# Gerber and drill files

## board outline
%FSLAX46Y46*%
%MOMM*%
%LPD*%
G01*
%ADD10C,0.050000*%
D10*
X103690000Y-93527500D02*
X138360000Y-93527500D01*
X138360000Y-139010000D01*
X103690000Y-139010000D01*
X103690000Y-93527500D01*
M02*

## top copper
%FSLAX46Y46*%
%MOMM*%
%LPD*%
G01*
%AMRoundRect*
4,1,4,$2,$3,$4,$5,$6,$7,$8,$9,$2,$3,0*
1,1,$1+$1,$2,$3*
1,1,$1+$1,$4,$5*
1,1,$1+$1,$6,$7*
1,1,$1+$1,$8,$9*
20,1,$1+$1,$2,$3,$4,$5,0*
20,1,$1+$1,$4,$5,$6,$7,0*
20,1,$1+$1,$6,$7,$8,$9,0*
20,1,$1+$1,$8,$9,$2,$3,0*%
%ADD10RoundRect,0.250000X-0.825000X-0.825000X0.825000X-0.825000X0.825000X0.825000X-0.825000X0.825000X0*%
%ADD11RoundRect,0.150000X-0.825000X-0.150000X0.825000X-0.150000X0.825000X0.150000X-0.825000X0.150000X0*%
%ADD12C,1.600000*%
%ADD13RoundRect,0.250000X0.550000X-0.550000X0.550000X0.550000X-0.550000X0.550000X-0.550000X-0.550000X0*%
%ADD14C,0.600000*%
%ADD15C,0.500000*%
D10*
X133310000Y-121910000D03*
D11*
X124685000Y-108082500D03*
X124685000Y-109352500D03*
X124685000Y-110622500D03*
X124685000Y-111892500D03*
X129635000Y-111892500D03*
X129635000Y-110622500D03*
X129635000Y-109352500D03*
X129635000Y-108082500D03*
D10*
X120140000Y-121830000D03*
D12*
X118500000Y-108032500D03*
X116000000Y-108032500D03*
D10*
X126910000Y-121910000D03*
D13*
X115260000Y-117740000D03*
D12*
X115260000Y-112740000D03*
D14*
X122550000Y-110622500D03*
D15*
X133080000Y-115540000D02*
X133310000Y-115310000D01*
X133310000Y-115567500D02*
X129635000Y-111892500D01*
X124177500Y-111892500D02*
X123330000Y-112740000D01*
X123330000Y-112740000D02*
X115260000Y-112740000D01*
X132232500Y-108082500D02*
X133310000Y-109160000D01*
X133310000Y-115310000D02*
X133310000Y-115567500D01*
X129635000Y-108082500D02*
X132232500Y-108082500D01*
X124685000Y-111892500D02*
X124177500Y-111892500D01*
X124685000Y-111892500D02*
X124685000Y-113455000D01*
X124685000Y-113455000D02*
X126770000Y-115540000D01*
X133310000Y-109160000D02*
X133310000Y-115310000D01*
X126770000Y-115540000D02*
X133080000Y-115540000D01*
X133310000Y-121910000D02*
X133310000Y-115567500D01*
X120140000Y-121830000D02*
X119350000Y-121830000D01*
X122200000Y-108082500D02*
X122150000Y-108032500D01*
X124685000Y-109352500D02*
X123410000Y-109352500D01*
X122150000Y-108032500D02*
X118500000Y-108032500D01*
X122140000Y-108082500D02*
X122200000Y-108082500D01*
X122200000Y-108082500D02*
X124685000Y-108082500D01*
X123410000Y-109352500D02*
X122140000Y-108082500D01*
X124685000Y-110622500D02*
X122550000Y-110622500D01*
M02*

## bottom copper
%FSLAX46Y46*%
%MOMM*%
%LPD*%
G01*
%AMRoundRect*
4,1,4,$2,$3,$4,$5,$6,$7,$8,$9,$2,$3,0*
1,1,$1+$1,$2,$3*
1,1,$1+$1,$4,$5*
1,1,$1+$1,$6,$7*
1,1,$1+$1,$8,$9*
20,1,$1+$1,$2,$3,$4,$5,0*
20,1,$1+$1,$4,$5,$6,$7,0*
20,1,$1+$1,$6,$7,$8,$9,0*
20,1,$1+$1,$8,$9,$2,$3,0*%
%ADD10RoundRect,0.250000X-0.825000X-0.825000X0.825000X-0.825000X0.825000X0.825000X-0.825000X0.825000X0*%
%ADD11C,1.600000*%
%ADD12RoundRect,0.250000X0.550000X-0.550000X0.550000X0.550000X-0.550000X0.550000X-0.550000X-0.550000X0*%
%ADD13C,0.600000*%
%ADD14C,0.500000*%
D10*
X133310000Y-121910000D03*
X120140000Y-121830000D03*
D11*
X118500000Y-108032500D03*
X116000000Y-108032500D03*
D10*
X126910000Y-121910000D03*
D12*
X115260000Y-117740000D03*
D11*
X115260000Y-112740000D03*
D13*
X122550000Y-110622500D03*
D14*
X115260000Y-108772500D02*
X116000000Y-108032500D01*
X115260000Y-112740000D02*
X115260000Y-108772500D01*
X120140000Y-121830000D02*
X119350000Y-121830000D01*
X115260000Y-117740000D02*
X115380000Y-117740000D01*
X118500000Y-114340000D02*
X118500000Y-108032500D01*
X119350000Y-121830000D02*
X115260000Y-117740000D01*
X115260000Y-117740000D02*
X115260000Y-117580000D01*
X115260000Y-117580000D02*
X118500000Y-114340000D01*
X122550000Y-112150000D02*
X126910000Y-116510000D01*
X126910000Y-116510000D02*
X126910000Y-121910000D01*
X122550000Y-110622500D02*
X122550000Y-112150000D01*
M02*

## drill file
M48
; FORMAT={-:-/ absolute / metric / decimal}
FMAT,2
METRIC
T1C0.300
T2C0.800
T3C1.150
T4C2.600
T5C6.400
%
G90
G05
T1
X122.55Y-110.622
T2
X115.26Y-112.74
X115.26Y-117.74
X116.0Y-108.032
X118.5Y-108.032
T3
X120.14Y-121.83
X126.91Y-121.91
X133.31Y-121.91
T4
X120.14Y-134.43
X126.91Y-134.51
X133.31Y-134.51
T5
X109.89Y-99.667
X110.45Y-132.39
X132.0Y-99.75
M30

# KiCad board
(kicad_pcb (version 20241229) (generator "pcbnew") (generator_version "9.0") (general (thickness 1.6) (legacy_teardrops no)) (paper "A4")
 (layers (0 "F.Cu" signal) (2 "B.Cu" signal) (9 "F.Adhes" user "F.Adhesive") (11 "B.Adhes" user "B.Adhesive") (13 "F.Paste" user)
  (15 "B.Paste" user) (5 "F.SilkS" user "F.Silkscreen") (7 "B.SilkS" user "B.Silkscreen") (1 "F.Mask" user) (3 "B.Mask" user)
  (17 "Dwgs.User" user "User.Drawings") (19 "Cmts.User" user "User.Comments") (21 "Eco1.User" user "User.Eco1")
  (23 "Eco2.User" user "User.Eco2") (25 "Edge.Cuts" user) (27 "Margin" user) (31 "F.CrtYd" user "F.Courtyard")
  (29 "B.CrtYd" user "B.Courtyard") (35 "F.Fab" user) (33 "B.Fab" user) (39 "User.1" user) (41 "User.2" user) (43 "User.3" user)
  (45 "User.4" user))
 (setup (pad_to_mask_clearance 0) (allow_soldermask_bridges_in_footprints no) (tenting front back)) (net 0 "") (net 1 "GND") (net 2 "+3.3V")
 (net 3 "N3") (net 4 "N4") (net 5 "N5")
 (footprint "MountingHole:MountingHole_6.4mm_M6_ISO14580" (layer "F.Cu") (at 132 99.75)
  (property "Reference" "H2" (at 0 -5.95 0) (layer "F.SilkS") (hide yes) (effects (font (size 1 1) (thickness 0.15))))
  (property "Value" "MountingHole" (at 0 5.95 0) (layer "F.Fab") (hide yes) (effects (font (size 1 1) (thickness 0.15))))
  (pad "" np_thru_hole circle (at 0 0) (size 6.4 6.4) (drill 6.4) (layers "*.Cu" "*.Mask")))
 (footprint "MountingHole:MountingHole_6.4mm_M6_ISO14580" (layer "F.Cu") (at 109.89 99.6675)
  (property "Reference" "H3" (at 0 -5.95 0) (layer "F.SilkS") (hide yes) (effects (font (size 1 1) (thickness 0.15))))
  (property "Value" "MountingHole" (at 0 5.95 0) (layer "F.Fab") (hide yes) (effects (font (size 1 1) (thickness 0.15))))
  (pad "" np_thru_hole circle (at 0 0) (size 6.4 6.4) (drill 6.4) (layers "*.Cu" "*.Mask")))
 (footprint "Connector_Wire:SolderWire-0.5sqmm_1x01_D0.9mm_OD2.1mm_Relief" (layer "F.Cu") (at 133.31 121.91)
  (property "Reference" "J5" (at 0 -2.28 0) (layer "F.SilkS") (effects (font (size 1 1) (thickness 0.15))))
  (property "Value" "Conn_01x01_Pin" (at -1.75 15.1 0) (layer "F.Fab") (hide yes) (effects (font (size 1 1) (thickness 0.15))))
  (pad "" np_thru_hole circle (at 0 12.6) (size 2.6 2.6) (drill 2.6) (layers "*.Cu" "*.Mask"))
  (pad "1" thru_hole roundrect (at 0 0) (size 2.15 2.15) (drill 1.15) (layers "*.Cu" "*.Mask") (remove_unused_layers no)
   (roundrect_rratio 0.116279) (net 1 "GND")))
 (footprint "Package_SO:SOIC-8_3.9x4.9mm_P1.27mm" (layer "F.Cu") (at 127.16 109.9875)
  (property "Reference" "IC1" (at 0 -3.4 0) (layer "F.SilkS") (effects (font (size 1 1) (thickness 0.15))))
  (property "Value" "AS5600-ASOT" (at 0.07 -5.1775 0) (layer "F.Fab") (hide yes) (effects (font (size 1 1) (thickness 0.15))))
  (pad "1" smd roundrect (at -2.475 -1.905) (size 1.95 0.6) (layers "F.Cu" "F.Mask" "F.Paste") (roundrect_rratio 0.25) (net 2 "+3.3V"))
  (pad "2" smd roundrect (at -2.475 -0.635) (size 1.95 0.6) (layers "F.Cu" "F.Mask" "F.Paste") (roundrect_rratio 0.25) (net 2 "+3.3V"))
  (pad "3" smd roundrect (at -2.475 0.635) (size 1.95 0.6) (layers "F.Cu" "F.Mask" "F.Paste") (roundrect_rratio 0.25) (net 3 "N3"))
  (pad "4" smd roundrect (at -2.475 1.905) (size 1.95 0.6) (layers "F.Cu" "F.Mask" "F.Paste") (roundrect_rratio 0.25) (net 1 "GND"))
  (pad "5" smd roundrect (at 2.475 1.905) (size 1.95 0.6) (layers "F.Cu" "F.Mask" "F.Paste") (roundrect_rratio 0.25) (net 1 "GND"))
  (pad "6" smd roundrect (at 2.475 0.635) (size 1.95 0.6) (layers "F.Cu" "F.Mask" "F.Paste") (roundrect_rratio 0.25) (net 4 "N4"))
  (pad "7" smd roundrect (at 2.475 -0.635) (size 1.95 0.6) (layers "F.Cu" "F.Mask" "F.Paste") (roundrect_rratio 0.25) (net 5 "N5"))
  (pad "8" smd roundrect (at 2.475 -1.905) (size 1.95 0.6) (layers "F.Cu" "F.Mask" "F.Paste") (roundrect_rratio 0.25) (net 1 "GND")))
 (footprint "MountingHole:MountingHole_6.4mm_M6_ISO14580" (layer "F.Cu") (at 110.45 132.39)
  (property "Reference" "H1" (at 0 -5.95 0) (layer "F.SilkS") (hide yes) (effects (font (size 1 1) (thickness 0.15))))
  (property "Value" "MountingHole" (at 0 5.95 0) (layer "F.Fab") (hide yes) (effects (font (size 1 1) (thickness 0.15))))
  (pad "" np_thru_hole circle (at 0 0) (size 6.4 6.4) (drill 6.4) (layers "*.Cu" "*.Mask")))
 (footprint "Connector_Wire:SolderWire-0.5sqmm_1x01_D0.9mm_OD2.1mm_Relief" (layer "F.Cu") (at 120.14 121.83)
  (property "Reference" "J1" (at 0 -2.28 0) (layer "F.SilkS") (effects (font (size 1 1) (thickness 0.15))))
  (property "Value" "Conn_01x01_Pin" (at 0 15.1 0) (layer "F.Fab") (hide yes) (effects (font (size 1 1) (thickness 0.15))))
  (pad "" np_thru_hole circle (at 0 12.6) (size 2.6 2.6) (drill 2.6) (layers "*.Cu" "*.Mask"))
  (pad "1" thru_hole roundrect (at 0 0) (size 2.15 2.15) (drill 1.15) (layers "*.Cu" "*.Mask") (remove_unused_layers no)
   (roundrect_rratio 0.116279) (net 2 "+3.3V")))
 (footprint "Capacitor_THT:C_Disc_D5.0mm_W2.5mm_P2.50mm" (layer "F.Cu") (at 118.5 108.0325 180)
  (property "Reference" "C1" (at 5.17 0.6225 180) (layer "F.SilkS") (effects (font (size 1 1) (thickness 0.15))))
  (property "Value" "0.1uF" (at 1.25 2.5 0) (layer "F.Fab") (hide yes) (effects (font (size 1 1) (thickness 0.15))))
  (pad "1" thru_hole circle (at 0 0 180) (size 1.6 1.6) (drill 0.8) (layers "*.Cu" "*.Mask") (remove_unused_layers no) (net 2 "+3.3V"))
  (pad "2" thru_hole circle (at 2.5 0 180) (size 1.6 1.6) (drill 0.8) (layers "*.Cu" "*.Mask") (remove_unused_layers no) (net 1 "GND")))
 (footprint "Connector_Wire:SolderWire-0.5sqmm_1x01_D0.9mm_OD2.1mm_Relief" (layer "F.Cu") (at 126.91 121.91)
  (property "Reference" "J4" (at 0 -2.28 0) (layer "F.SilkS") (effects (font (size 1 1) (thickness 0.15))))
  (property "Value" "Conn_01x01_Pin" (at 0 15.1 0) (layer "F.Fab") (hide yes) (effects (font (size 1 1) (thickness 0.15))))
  (pad "" np_thru_hole circle (at 0 12.6) (size 2.6 2.6) (drill 2.6) (layers "*.Cu" "*.Mask"))
  (pad "1" thru_hole roundrect (at 0 0) (size 2.15 2.15) (drill 1.15) (layers "*.Cu" "*.Mask") (remove_unused_layers no)
   (roundrect_rratio 0.116279) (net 3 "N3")))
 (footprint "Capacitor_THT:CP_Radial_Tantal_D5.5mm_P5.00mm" (layer "F.Cu") (at 115.26 117.74 90)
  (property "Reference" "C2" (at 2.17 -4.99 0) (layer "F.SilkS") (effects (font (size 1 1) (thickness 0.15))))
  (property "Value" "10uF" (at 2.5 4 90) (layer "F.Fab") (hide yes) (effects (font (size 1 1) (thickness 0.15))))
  (pad "1" thru_hole roundrect (at 0 0 90) (size 1.6 1.6) (drill 0.8) (layers "*.Cu" "*.Mask") (remove_unused_layers no)
   (roundrect_rratio 0.15625) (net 2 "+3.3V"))
  (pad "2" thru_hole circle (at 5 0 90) (size 1.6 1.6) (drill 0.8) (layers "*.Cu" "*.Mask") (remove_unused_layers no) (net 1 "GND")))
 (gr_rect (start 103.69 93.5275) (end 138.36 139.01) (stroke (width 0.05) (type default)) (fill no) (layer "Edge.Cuts"))
 (segment (start 133.08 115.54) (end 133.31 115.31) (width 0.5) (layer "F.Cu") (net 1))
 (segment (start 133.31 115.5675) (end 129.635 111.8925) (width 0.5) (layer "F.Cu") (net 1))
 (segment (start 124.1775 111.8925) (end 123.33 112.74) (width 0.5) (layer "F.Cu") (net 1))
 (segment (start 123.33 112.74) (end 115.26 112.74) (width 0.5) (layer "F.Cu") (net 1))
 (segment (start 132.2325 108.0825) (end 133.31 109.16) (width 0.5) (layer "F.Cu") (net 1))
 (segment (start 133.31 115.31) (end 133.31 115.5675) (width 0.5) (layer "F.Cu") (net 1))
 (segment (start 129.635 108.0825) (end 132.2325 108.0825) (width 0.5) (layer "F.Cu") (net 1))
 (segment (start 124.685 111.8925) (end 124.1775 111.8925) (width 0.5) (layer "F.Cu") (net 1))
 (segment (start 124.685 111.8925) (end 124.685 113.455) (width 0.5) (layer "F.Cu") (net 1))
 (segment (start 124.685 113.455) (end 126.77 115.54) (width 0.5) (layer "F.Cu") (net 1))
 (segment (start 133.31 109.16) (end 133.31 115.31) (width 0.5) (layer "F.Cu") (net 1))
 (segment (start 126.77 115.54) (end 133.08 115.54) (width 0.5) (layer "F.Cu") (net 1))
 (segment (start 133.31 121.91) (end 133.31 115.5675) (width 0.5) (layer "F.Cu") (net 1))
 (segment (start 115.26 108.7725) (end 116 108.0325) (width 0.5) (layer "B.Cu") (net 1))
 (segment (start 115.26 112.74) (end 115.26 108.7725) (width 0.5) (layer "B.Cu") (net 1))
 (segment (start 120.14 121.83) (end 119.35 121.83) (width 0.5) (layer "F.Cu") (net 2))
 (segment (start 122.2 108.0825) (end 122.15 108.0325) (width 0.5) (layer "F.Cu") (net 2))
 (segment (start 124.685 109.3525) (end 123.41 109.3525) (width 0.5) (layer "F.Cu") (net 2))
 (segment (start 122.15 108.0325) (end 118.5 108.0325) (width 0.5) (layer "F.Cu") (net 2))
 (segment (start 122.14 108.0825) (end 122.2 108.0825) (width 0.5) (layer "F.Cu") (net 2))
 (segment (start 122.2 108.0825) (end 124.685 108.0825) (width 0.5) (layer "F.Cu") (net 2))
 (segment (start 123.41 109.3525) (end 122.14 108.0825) (width 0.5) (layer "F.Cu") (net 2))
 (segment (start 120.14 121.83) (end 119.35 121.83) (width 0.5) (layer "B.Cu") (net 2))
 (segment (start 115.26 117.74) (end 115.38 117.74) (width 0.5) (layer "B.Cu") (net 2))
 (segment (start 118.5 114.34) (end 118.5 108.0325) (width 0.5) (layer "B.Cu") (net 2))
 (segment (start 119.35 121.83) (end 115.26 117.74) (width 0.5) (layer "B.Cu") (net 2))
 (segment (start 115.26 117.74) (end 115.26 117.58) (width 0.5) (layer "B.Cu") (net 2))
 (segment (start 115.26 117.58) (end 118.5 114.34) (width 0.5) (layer "B.Cu") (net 2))
 (segment (start 124.685 110.6225) (end 122.55 110.6225) (width 0.5) (layer "F.Cu") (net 3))
 (via (at 122.55 110.6225) (size 0.6) (drill 0.3) (layers "F.Cu" "B.Cu") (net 3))
 (segment (start 122.55 112.15) (end 126.91 116.51) (width 0.5) (layer "B.Cu") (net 3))
 (segment (start 126.91 116.51) (end 126.91 121.91) (width 0.5) (layer "B.Cu") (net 3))
 (segment (start 122.55 110.6225) (end 122.55 112.15) (width 0.5) (layer "B.Cu") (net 3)))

